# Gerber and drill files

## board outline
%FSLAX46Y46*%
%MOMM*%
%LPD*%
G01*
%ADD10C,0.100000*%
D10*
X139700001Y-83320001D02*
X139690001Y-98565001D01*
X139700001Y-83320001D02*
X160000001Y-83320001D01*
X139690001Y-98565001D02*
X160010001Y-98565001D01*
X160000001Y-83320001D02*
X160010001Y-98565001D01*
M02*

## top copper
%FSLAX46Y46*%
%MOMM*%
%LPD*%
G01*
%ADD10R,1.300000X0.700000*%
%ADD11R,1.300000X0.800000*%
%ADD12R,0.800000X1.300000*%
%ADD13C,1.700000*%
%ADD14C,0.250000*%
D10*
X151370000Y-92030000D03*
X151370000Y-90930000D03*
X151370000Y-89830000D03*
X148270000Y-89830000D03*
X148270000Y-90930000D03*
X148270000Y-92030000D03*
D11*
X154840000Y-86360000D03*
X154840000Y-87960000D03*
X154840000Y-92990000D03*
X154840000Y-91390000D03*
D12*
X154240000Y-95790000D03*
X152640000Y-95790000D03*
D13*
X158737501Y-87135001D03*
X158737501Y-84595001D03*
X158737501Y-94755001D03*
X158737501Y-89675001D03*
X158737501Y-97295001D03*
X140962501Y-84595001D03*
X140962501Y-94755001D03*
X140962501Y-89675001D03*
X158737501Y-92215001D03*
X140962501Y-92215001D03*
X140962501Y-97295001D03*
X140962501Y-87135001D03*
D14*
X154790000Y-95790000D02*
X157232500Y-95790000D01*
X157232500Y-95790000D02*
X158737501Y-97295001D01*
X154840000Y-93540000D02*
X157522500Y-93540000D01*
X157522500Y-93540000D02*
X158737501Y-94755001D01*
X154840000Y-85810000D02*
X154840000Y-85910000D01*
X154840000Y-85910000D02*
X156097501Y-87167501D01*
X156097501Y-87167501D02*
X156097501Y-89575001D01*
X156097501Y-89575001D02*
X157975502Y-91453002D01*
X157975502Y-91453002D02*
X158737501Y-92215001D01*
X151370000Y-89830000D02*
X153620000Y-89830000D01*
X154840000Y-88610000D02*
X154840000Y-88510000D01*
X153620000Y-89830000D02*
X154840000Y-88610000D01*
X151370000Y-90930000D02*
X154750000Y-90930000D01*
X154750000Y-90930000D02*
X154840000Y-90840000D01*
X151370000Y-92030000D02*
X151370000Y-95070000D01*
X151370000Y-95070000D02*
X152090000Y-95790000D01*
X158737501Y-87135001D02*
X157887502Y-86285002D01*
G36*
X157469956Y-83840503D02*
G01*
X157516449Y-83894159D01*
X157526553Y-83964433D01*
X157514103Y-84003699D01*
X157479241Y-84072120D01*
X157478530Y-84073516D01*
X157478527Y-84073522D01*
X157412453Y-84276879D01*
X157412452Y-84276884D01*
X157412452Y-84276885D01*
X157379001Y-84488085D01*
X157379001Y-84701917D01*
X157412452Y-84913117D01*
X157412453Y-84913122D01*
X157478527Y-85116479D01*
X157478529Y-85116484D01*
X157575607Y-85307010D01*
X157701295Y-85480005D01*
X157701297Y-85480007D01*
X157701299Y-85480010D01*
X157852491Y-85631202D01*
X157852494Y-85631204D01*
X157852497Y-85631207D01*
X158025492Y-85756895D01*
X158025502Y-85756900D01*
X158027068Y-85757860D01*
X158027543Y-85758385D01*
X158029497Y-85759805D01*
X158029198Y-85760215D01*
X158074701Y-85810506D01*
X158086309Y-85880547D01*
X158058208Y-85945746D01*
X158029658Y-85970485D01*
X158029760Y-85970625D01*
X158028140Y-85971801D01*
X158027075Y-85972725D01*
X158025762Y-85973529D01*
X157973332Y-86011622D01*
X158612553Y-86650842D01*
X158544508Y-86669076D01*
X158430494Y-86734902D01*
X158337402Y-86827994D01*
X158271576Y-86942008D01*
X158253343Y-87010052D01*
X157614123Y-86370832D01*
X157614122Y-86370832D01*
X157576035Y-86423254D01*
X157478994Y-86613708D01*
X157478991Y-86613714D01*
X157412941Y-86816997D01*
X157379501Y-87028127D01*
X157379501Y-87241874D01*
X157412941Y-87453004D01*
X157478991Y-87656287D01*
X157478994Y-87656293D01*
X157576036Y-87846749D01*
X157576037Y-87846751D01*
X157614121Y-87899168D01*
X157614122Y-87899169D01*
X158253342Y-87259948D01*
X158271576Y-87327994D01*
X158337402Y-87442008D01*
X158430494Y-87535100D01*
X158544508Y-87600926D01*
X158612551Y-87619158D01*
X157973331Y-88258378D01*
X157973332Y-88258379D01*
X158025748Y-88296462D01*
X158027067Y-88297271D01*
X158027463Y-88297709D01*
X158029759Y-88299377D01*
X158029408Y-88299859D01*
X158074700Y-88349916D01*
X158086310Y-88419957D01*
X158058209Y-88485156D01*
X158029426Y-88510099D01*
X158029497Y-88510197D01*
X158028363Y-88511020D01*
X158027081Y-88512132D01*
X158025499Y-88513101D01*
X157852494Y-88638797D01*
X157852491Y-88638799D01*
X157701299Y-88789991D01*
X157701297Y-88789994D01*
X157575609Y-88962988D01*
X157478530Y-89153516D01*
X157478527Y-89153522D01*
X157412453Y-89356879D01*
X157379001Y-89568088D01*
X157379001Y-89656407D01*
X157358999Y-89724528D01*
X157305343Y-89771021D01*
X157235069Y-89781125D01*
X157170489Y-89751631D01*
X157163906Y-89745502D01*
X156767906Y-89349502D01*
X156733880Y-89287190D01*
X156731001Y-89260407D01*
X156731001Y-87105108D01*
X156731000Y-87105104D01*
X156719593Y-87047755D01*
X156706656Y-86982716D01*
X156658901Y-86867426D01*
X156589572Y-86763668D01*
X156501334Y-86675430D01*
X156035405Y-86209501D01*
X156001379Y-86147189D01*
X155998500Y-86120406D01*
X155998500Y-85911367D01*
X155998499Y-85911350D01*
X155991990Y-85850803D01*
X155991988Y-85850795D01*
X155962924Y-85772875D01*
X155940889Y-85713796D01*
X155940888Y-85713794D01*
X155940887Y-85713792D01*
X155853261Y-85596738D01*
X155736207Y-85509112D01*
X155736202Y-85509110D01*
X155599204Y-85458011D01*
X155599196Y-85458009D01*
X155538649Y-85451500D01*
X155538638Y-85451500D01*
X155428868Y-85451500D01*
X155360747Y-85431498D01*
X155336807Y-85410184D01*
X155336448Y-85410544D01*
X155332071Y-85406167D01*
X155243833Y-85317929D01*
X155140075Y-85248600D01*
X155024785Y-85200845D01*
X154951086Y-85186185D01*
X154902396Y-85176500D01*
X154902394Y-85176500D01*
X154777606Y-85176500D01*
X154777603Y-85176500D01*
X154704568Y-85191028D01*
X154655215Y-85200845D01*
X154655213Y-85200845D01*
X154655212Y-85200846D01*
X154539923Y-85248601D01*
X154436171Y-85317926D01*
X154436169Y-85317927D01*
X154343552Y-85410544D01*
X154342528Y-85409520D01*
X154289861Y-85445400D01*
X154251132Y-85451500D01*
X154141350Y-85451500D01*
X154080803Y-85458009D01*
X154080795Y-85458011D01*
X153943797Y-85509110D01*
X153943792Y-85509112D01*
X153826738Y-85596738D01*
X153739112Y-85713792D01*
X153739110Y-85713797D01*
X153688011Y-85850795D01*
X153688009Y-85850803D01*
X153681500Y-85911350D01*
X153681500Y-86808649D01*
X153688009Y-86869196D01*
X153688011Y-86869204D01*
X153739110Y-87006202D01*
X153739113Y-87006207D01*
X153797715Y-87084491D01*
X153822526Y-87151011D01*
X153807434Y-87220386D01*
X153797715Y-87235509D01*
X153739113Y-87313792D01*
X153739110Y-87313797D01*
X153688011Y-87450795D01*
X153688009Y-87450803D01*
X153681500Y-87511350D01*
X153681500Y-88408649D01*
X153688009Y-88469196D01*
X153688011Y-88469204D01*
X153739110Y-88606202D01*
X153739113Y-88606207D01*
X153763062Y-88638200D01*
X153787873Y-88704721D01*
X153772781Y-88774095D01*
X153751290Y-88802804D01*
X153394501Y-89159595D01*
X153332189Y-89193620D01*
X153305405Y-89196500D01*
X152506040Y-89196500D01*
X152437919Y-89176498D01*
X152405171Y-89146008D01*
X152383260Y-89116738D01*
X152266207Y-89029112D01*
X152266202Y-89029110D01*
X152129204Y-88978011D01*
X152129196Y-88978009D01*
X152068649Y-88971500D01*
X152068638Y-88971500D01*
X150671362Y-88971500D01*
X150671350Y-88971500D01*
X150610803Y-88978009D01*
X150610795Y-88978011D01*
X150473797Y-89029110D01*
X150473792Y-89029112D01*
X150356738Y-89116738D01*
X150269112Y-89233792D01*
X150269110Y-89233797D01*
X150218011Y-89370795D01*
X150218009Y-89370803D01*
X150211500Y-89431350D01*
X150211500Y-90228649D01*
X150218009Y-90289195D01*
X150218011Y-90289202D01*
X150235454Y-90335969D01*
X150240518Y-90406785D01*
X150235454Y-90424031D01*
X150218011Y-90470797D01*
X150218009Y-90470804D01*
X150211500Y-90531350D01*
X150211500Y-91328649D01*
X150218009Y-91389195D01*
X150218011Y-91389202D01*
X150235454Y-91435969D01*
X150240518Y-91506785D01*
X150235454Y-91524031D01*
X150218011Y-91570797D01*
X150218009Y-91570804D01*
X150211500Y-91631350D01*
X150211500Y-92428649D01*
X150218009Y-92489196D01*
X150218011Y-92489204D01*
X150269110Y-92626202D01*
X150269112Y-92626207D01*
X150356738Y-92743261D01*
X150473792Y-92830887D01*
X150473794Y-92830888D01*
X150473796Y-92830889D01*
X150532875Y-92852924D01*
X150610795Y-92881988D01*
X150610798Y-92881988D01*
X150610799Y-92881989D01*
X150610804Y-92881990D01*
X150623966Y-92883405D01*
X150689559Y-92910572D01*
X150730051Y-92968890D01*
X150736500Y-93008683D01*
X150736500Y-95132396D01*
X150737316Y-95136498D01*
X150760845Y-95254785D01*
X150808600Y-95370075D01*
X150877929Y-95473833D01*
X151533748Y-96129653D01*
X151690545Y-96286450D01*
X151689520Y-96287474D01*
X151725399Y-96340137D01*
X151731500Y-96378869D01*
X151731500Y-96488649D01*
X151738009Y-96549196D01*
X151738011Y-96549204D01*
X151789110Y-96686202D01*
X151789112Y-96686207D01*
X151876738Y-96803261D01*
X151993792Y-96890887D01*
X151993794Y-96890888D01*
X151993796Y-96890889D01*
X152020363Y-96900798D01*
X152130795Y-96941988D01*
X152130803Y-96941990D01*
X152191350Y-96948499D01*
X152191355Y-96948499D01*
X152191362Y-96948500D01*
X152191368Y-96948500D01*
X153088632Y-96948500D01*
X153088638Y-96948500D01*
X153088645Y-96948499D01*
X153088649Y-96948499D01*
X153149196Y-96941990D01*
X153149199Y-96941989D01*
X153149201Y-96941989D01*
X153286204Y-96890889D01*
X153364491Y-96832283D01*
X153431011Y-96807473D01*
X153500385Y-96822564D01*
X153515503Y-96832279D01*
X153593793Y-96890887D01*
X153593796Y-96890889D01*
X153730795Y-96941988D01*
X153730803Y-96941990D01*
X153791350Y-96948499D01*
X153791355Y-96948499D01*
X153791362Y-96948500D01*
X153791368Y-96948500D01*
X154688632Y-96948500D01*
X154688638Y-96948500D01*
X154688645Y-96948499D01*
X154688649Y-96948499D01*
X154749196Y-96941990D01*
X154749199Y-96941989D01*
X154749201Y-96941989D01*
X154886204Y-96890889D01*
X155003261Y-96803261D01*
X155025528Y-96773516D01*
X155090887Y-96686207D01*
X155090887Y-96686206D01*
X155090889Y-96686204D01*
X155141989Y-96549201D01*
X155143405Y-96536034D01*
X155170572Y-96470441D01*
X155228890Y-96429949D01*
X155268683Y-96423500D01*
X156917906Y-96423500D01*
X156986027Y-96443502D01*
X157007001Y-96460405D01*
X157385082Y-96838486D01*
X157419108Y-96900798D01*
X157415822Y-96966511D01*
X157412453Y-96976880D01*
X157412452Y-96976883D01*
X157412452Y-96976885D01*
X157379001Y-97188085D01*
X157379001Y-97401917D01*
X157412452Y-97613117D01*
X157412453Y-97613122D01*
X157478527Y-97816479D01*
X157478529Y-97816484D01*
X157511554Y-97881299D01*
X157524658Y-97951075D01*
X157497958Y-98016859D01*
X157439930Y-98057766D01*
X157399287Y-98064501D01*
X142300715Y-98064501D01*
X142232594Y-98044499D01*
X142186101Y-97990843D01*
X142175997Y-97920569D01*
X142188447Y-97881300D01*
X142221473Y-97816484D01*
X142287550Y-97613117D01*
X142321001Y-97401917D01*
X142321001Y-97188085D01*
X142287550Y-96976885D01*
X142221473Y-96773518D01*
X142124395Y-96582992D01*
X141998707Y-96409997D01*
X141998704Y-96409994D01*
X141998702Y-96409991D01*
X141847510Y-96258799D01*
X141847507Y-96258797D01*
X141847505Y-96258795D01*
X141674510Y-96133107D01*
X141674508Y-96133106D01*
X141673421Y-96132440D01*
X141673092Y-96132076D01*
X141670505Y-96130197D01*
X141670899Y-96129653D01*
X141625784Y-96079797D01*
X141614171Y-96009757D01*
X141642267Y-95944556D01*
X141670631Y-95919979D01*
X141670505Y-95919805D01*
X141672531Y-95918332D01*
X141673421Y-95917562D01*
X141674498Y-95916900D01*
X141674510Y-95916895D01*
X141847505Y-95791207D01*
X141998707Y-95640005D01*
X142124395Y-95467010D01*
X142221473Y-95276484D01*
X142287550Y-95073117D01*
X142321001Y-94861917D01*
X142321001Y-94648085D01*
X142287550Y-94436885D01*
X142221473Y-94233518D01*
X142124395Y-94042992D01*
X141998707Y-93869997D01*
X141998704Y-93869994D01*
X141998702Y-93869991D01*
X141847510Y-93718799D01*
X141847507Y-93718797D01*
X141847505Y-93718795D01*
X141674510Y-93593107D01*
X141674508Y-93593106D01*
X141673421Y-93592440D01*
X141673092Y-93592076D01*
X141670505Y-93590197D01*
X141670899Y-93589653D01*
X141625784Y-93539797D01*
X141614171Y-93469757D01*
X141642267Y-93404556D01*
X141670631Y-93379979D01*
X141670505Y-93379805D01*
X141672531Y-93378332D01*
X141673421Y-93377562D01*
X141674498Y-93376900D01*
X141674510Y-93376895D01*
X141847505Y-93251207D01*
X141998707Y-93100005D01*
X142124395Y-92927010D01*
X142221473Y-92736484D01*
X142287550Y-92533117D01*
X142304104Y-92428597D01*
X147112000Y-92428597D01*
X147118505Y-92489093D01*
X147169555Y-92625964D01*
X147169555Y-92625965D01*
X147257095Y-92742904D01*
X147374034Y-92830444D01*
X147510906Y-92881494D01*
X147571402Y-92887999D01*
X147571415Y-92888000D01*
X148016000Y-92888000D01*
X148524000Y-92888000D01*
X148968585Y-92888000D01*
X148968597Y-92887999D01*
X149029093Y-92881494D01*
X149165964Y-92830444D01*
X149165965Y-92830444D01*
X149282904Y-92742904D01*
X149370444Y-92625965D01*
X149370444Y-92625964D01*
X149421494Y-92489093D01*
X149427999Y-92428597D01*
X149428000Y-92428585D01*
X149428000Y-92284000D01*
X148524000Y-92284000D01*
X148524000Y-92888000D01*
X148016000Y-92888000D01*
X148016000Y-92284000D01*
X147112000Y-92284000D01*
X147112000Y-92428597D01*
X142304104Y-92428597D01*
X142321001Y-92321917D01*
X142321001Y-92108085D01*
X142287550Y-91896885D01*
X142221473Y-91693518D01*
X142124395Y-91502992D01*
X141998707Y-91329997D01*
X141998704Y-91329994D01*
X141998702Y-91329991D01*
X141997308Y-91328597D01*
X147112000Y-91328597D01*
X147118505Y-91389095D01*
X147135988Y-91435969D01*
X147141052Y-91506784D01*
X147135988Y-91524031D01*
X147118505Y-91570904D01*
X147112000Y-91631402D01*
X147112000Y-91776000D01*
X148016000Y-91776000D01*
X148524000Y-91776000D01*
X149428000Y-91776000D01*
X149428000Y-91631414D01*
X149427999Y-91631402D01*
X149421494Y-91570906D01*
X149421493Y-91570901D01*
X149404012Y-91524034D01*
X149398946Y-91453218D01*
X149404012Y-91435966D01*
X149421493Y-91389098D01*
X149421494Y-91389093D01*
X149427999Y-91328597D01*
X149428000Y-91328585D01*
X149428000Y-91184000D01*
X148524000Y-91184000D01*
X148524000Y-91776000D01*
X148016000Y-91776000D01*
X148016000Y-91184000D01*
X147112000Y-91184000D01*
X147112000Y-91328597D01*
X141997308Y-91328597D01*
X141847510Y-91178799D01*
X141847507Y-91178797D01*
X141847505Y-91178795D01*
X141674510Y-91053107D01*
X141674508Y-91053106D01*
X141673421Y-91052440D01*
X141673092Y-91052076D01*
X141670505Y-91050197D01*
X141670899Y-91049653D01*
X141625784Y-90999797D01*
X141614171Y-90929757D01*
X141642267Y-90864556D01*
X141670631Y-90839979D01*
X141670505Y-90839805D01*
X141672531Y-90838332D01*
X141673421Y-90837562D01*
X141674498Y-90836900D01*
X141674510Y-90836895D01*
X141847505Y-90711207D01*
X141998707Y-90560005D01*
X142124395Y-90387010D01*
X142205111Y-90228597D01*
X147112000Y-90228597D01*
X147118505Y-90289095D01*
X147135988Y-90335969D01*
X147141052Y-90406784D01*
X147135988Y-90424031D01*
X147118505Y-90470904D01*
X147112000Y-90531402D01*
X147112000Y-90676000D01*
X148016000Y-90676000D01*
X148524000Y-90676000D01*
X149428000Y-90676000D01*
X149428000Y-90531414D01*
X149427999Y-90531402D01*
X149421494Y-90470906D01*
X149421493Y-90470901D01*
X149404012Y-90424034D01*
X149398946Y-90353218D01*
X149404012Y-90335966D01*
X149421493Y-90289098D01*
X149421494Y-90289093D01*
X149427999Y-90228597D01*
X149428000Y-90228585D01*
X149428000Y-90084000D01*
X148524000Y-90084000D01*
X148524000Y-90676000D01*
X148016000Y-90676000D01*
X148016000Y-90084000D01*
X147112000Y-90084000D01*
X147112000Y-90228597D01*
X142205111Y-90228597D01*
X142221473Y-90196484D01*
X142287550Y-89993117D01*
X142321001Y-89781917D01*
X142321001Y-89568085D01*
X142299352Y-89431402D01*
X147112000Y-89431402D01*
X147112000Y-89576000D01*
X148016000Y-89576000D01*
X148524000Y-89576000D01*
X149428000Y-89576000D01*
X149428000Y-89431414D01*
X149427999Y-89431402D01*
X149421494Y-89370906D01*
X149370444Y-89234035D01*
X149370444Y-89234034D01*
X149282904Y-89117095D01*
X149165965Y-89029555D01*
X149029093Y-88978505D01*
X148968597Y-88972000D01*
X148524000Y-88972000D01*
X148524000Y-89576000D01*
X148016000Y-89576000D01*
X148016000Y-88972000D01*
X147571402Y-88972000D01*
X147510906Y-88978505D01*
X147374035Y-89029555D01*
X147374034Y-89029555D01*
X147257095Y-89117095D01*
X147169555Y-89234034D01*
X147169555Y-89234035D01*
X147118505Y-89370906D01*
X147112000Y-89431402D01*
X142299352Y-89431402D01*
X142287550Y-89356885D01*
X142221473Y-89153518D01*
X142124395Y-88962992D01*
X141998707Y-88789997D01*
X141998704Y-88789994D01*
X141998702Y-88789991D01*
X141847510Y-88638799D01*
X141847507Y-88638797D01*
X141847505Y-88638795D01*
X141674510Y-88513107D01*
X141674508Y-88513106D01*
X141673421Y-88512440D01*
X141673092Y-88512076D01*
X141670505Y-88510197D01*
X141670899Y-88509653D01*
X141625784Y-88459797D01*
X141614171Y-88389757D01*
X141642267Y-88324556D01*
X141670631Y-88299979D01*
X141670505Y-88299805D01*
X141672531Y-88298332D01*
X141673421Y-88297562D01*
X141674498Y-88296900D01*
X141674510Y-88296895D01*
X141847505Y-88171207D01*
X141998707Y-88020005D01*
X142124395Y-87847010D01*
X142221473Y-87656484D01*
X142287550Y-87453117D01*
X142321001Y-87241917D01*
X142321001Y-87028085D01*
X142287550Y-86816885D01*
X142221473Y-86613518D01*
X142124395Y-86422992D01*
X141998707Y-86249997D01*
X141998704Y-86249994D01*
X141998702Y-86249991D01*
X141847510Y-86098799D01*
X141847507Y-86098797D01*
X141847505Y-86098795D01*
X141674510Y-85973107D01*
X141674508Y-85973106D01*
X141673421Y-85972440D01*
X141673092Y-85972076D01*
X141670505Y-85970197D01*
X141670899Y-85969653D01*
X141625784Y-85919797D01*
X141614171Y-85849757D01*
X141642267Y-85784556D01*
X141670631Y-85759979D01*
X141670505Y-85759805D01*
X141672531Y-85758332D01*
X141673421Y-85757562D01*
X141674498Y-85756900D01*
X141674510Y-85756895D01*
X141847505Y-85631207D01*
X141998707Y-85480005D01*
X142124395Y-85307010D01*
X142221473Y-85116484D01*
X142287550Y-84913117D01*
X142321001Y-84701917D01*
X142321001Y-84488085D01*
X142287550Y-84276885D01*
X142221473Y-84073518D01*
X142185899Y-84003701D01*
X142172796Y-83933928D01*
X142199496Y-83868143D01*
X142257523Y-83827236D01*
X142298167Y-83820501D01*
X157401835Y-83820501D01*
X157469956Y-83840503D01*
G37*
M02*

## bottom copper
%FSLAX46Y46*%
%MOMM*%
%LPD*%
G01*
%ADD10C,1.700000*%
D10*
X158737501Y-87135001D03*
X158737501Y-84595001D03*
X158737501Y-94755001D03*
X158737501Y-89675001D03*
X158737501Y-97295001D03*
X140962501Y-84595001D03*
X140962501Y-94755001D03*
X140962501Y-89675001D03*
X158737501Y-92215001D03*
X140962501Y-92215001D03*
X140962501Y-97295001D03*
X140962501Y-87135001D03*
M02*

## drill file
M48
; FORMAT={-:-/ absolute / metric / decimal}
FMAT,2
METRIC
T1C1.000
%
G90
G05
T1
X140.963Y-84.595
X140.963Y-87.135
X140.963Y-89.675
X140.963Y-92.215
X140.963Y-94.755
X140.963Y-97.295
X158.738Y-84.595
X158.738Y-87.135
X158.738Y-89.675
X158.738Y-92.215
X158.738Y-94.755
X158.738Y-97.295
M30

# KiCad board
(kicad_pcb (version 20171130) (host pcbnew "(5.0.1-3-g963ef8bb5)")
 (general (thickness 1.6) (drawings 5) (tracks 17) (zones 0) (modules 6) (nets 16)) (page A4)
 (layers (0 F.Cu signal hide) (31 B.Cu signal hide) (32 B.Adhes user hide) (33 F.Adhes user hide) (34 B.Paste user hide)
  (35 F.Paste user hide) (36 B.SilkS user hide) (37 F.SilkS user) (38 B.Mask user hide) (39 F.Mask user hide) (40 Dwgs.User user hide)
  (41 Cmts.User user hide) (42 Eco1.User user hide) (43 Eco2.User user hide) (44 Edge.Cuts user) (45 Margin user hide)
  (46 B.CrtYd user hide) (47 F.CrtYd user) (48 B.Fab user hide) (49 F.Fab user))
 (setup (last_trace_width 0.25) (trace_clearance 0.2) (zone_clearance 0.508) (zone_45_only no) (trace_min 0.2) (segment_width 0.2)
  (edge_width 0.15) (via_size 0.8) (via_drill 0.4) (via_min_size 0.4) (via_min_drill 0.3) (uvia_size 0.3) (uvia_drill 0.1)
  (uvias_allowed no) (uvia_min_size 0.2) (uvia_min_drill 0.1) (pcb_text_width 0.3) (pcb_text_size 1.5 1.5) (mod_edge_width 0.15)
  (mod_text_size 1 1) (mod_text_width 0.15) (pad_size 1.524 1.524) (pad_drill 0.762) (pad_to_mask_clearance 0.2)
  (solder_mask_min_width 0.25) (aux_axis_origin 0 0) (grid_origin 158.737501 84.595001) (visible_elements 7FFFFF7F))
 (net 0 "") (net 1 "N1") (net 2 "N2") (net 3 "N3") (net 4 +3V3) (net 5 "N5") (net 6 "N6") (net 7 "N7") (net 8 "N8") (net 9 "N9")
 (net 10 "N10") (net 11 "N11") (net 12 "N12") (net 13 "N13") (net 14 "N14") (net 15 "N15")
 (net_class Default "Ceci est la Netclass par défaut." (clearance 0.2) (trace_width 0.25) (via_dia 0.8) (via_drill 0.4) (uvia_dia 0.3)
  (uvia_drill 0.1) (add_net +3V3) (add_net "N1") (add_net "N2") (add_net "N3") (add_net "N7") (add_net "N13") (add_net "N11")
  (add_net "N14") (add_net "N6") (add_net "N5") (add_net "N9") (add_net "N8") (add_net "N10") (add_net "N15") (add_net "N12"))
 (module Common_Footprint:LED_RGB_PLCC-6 (layer F.Cu) (at 149.82 90.93 180)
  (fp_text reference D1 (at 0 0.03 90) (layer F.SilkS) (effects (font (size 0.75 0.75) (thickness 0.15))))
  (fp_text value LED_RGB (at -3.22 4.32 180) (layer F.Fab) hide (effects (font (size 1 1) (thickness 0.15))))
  (pad 1 smd rect (at -1.55 -1.1 270) (size 0.7 1.3) (layers F.Cu F.Paste F.Mask) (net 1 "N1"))
  (pad 2 smd rect (at -1.55 0 270) (size 0.7 1.3) (layers F.Cu F.Paste F.Mask) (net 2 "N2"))
  (pad 3 smd rect (at -1.55 1.1 270) (size 0.7 1.3) (layers F.Cu F.Paste F.Mask) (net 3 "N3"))
  (pad 4 smd rect (at 1.55 1.1 270) (size 0.7 1.3) (layers F.Cu F.Paste F.Mask) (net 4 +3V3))
  (pad 5 smd rect (at 1.55 0 270) (size 0.7 1.3) (layers F.Cu F.Paste F.Mask) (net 4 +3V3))
  (pad 6 smd rect (at 1.55 -1.1 270) (size 0.7 1.3) (layers F.Cu F.Paste F.Mask) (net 4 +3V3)))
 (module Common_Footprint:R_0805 (layer F.Cu) (at 154.84 87.16 270)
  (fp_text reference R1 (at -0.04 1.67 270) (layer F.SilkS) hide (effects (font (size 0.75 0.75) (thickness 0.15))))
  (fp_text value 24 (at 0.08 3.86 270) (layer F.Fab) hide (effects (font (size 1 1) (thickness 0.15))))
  (pad 1 smd rect (at -0.8 0 270) (size 0.8 1.3) (layers F.Cu F.Paste F.Mask) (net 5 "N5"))
  (pad 2 smd rect (at 0.8 0 270) (size 0.8 1.3) (layers F.Cu F.Paste F.Mask) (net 3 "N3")))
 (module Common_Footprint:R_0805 (layer F.Cu) (at 154.84 92.19 90)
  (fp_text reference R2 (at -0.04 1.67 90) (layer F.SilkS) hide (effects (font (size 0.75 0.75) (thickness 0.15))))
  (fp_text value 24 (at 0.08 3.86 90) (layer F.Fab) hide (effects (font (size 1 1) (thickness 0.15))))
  (pad 1 smd rect (at -0.8 0 90) (size 0.8 1.3) (layers F.Cu F.Paste F.Mask) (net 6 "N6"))
  (pad 2 smd rect (at 0.8 0 90) (size 0.8 1.3) (layers F.Cu F.Paste F.Mask) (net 2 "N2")))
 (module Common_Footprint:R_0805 (layer F.Cu) (at 153.44 95.79 180)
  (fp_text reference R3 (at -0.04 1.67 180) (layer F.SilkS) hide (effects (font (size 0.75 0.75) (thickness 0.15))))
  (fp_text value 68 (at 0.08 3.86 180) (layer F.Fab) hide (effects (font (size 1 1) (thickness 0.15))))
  (pad 1 smd rect (at -0.8 0 180) (size 0.8 1.3) (layers F.Cu F.Paste F.Mask) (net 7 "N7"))
  (pad 2 smd rect (at 0.8 0 180) (size 0.8 1.3) (layers F.Cu F.Paste F.Mask) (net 1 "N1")))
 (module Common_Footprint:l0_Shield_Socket (layer F.Cu) (at 149.850001 90.945001)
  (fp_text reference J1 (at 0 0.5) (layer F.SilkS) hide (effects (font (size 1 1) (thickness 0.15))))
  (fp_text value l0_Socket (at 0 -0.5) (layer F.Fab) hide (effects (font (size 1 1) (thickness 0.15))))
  (fp_line (start -10.15 -7.625) (end -10.16 7.62) (layer Edge.Cuts) (width 0.1))
  (fp_line (start -10.15 -7.625) (end 10.15 -7.625) (layer Edge.Cuts) (width 0.1))
  (fp_line (start -10.16 7.62) (end 10.16 7.62) (layer Edge.Cuts) (width 0.1))
  (fp_line (start 10.15 -7.625) (end 10.16 7.62) (layer Edge.Cuts) (width 0.1))
  (pad 5 thru_hole circle (at 8.8875 -3.81 270) (size 1.7 1.7) (drill 1) (layers *.Cu *.Mask) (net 4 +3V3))
  (pad 6 thru_hole circle (at 8.8875 -6.35 270) (size 1.7 1.7) (drill 1) (layers *.Cu *.Mask) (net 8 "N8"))
  (pad 2 thru_hole circle (at 8.8875 3.81 270) (size 1.7 1.7) (drill 1) (layers *.Cu *.Mask) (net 6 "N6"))
  (pad 4 thru_hole circle (at 8.8875 -1.27 270) (size 1.7 1.7) (drill 1) (layers *.Cu *.Mask) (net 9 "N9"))
  (pad 1 thru_hole circle (at 8.8875 6.35 270) (size 1.7 1.7) (drill 1) (layers *.Cu *.Mask) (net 7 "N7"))
  (pad 7 thru_hole circle (at -8.8875 -6.35 270) (size 1.7 1.7) (drill 1) (layers *.Cu *.Mask) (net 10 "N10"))
  (pad 11 thru_hole circle (at -8.8875 3.81 270) (size 1.7 1.7) (drill 1) (layers *.Cu *.Mask) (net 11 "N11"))
  (pad 9 thru_hole circle (at -8.8875 -1.27 270) (size 1.7 1.7) (drill 1) (layers *.Cu *.Mask) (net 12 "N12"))
  (pad 3 thru_hole circle (at 8.8875 1.27 270) (size 1.7 1.7) (drill 1) (layers *.Cu *.Mask) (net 5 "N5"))
  (pad 10 thru_hole circle (at -8.8875 1.27 270) (size 1.7 1.7) (drill 1) (layers *.Cu *.Mask) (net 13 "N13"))
  (pad 12 thru_hole circle (at -8.8875 6.35 270) (size 1.7 1.7) (drill 1) (layers *.Cu *.Mask) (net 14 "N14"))
  (pad 8 thru_hole circle (at -8.8875 -3.81 270) (size 1.7 1.7) (drill 1) (layers *.Cu *.Mask) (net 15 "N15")))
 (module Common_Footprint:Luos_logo (layer F.Cu) (at 145.227501 91.715001 270)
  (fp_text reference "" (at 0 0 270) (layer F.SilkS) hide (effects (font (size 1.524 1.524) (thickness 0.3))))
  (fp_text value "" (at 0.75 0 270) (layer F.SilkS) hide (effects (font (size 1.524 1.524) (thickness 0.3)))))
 (segment (start 154.79 95.79) (end 157.2325 95.79) (width 0.25) (layer F.Cu) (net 7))
 (segment (start 157.2325 95.79) (end 158.737501 97.295001) (width 0.25) (layer F.Cu) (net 7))
 (segment (start 154.84 93.54) (end 157.5225 93.54) (width 0.25) (layer F.Cu) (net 6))
 (segment (start 157.5225 93.54) (end 158.737501 94.755001) (width 0.25) (layer F.Cu) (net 6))
 (segment (start 154.84 85.81) (end 154.84 85.91) (width 0.25) (layer F.Cu) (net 5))
 (segment (start 154.84 85.91) (end 156.097501 87.167501) (width 0.25) (layer F.Cu) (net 5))
 (segment (start 156.097501 87.167501) (end 156.097501 89.575001) (width 0.25) (layer F.Cu) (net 5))
 (segment (start 156.097501 89.575001) (end 157.975502 91.453002) (width 0.25) (layer F.Cu) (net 5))
 (segment (start 157.975502 91.453002) (end 158.737501 92.215001) (width 0.25) (layer F.Cu) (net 5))
 (segment (start 151.37 89.83) (end 153.62 89.83) (width 0.25) (layer F.Cu) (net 3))
 (segment (start 154.84 88.61) (end 154.84 88.51) (width 0.25) (layer F.Cu) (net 3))
 (segment (start 153.62 89.83) (end 154.84 88.61) (width 0.25) (layer F.Cu) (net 3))
 (segment (start 151.37 90.93) (end 154.75 90.93) (width 0.25) (layer F.Cu) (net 2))
 (segment (start 154.75 90.93) (end 154.84 90.84) (width 0.25) (layer F.Cu) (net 2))
 (segment (start 151.37 92.03) (end 151.37 95.07) (width 0.25) (layer F.Cu) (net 1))
 (segment (start 151.37 95.07) (end 152.09 95.79) (width 0.25) (layer F.Cu) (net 1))
 (segment (start 158.737501 87.135001) (end 157.887502 86.285002) (width 0.25) (layer F.Cu) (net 4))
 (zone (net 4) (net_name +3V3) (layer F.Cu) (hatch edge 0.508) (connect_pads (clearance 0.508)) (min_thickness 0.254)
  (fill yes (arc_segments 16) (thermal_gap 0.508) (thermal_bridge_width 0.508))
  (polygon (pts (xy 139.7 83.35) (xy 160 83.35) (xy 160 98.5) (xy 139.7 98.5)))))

